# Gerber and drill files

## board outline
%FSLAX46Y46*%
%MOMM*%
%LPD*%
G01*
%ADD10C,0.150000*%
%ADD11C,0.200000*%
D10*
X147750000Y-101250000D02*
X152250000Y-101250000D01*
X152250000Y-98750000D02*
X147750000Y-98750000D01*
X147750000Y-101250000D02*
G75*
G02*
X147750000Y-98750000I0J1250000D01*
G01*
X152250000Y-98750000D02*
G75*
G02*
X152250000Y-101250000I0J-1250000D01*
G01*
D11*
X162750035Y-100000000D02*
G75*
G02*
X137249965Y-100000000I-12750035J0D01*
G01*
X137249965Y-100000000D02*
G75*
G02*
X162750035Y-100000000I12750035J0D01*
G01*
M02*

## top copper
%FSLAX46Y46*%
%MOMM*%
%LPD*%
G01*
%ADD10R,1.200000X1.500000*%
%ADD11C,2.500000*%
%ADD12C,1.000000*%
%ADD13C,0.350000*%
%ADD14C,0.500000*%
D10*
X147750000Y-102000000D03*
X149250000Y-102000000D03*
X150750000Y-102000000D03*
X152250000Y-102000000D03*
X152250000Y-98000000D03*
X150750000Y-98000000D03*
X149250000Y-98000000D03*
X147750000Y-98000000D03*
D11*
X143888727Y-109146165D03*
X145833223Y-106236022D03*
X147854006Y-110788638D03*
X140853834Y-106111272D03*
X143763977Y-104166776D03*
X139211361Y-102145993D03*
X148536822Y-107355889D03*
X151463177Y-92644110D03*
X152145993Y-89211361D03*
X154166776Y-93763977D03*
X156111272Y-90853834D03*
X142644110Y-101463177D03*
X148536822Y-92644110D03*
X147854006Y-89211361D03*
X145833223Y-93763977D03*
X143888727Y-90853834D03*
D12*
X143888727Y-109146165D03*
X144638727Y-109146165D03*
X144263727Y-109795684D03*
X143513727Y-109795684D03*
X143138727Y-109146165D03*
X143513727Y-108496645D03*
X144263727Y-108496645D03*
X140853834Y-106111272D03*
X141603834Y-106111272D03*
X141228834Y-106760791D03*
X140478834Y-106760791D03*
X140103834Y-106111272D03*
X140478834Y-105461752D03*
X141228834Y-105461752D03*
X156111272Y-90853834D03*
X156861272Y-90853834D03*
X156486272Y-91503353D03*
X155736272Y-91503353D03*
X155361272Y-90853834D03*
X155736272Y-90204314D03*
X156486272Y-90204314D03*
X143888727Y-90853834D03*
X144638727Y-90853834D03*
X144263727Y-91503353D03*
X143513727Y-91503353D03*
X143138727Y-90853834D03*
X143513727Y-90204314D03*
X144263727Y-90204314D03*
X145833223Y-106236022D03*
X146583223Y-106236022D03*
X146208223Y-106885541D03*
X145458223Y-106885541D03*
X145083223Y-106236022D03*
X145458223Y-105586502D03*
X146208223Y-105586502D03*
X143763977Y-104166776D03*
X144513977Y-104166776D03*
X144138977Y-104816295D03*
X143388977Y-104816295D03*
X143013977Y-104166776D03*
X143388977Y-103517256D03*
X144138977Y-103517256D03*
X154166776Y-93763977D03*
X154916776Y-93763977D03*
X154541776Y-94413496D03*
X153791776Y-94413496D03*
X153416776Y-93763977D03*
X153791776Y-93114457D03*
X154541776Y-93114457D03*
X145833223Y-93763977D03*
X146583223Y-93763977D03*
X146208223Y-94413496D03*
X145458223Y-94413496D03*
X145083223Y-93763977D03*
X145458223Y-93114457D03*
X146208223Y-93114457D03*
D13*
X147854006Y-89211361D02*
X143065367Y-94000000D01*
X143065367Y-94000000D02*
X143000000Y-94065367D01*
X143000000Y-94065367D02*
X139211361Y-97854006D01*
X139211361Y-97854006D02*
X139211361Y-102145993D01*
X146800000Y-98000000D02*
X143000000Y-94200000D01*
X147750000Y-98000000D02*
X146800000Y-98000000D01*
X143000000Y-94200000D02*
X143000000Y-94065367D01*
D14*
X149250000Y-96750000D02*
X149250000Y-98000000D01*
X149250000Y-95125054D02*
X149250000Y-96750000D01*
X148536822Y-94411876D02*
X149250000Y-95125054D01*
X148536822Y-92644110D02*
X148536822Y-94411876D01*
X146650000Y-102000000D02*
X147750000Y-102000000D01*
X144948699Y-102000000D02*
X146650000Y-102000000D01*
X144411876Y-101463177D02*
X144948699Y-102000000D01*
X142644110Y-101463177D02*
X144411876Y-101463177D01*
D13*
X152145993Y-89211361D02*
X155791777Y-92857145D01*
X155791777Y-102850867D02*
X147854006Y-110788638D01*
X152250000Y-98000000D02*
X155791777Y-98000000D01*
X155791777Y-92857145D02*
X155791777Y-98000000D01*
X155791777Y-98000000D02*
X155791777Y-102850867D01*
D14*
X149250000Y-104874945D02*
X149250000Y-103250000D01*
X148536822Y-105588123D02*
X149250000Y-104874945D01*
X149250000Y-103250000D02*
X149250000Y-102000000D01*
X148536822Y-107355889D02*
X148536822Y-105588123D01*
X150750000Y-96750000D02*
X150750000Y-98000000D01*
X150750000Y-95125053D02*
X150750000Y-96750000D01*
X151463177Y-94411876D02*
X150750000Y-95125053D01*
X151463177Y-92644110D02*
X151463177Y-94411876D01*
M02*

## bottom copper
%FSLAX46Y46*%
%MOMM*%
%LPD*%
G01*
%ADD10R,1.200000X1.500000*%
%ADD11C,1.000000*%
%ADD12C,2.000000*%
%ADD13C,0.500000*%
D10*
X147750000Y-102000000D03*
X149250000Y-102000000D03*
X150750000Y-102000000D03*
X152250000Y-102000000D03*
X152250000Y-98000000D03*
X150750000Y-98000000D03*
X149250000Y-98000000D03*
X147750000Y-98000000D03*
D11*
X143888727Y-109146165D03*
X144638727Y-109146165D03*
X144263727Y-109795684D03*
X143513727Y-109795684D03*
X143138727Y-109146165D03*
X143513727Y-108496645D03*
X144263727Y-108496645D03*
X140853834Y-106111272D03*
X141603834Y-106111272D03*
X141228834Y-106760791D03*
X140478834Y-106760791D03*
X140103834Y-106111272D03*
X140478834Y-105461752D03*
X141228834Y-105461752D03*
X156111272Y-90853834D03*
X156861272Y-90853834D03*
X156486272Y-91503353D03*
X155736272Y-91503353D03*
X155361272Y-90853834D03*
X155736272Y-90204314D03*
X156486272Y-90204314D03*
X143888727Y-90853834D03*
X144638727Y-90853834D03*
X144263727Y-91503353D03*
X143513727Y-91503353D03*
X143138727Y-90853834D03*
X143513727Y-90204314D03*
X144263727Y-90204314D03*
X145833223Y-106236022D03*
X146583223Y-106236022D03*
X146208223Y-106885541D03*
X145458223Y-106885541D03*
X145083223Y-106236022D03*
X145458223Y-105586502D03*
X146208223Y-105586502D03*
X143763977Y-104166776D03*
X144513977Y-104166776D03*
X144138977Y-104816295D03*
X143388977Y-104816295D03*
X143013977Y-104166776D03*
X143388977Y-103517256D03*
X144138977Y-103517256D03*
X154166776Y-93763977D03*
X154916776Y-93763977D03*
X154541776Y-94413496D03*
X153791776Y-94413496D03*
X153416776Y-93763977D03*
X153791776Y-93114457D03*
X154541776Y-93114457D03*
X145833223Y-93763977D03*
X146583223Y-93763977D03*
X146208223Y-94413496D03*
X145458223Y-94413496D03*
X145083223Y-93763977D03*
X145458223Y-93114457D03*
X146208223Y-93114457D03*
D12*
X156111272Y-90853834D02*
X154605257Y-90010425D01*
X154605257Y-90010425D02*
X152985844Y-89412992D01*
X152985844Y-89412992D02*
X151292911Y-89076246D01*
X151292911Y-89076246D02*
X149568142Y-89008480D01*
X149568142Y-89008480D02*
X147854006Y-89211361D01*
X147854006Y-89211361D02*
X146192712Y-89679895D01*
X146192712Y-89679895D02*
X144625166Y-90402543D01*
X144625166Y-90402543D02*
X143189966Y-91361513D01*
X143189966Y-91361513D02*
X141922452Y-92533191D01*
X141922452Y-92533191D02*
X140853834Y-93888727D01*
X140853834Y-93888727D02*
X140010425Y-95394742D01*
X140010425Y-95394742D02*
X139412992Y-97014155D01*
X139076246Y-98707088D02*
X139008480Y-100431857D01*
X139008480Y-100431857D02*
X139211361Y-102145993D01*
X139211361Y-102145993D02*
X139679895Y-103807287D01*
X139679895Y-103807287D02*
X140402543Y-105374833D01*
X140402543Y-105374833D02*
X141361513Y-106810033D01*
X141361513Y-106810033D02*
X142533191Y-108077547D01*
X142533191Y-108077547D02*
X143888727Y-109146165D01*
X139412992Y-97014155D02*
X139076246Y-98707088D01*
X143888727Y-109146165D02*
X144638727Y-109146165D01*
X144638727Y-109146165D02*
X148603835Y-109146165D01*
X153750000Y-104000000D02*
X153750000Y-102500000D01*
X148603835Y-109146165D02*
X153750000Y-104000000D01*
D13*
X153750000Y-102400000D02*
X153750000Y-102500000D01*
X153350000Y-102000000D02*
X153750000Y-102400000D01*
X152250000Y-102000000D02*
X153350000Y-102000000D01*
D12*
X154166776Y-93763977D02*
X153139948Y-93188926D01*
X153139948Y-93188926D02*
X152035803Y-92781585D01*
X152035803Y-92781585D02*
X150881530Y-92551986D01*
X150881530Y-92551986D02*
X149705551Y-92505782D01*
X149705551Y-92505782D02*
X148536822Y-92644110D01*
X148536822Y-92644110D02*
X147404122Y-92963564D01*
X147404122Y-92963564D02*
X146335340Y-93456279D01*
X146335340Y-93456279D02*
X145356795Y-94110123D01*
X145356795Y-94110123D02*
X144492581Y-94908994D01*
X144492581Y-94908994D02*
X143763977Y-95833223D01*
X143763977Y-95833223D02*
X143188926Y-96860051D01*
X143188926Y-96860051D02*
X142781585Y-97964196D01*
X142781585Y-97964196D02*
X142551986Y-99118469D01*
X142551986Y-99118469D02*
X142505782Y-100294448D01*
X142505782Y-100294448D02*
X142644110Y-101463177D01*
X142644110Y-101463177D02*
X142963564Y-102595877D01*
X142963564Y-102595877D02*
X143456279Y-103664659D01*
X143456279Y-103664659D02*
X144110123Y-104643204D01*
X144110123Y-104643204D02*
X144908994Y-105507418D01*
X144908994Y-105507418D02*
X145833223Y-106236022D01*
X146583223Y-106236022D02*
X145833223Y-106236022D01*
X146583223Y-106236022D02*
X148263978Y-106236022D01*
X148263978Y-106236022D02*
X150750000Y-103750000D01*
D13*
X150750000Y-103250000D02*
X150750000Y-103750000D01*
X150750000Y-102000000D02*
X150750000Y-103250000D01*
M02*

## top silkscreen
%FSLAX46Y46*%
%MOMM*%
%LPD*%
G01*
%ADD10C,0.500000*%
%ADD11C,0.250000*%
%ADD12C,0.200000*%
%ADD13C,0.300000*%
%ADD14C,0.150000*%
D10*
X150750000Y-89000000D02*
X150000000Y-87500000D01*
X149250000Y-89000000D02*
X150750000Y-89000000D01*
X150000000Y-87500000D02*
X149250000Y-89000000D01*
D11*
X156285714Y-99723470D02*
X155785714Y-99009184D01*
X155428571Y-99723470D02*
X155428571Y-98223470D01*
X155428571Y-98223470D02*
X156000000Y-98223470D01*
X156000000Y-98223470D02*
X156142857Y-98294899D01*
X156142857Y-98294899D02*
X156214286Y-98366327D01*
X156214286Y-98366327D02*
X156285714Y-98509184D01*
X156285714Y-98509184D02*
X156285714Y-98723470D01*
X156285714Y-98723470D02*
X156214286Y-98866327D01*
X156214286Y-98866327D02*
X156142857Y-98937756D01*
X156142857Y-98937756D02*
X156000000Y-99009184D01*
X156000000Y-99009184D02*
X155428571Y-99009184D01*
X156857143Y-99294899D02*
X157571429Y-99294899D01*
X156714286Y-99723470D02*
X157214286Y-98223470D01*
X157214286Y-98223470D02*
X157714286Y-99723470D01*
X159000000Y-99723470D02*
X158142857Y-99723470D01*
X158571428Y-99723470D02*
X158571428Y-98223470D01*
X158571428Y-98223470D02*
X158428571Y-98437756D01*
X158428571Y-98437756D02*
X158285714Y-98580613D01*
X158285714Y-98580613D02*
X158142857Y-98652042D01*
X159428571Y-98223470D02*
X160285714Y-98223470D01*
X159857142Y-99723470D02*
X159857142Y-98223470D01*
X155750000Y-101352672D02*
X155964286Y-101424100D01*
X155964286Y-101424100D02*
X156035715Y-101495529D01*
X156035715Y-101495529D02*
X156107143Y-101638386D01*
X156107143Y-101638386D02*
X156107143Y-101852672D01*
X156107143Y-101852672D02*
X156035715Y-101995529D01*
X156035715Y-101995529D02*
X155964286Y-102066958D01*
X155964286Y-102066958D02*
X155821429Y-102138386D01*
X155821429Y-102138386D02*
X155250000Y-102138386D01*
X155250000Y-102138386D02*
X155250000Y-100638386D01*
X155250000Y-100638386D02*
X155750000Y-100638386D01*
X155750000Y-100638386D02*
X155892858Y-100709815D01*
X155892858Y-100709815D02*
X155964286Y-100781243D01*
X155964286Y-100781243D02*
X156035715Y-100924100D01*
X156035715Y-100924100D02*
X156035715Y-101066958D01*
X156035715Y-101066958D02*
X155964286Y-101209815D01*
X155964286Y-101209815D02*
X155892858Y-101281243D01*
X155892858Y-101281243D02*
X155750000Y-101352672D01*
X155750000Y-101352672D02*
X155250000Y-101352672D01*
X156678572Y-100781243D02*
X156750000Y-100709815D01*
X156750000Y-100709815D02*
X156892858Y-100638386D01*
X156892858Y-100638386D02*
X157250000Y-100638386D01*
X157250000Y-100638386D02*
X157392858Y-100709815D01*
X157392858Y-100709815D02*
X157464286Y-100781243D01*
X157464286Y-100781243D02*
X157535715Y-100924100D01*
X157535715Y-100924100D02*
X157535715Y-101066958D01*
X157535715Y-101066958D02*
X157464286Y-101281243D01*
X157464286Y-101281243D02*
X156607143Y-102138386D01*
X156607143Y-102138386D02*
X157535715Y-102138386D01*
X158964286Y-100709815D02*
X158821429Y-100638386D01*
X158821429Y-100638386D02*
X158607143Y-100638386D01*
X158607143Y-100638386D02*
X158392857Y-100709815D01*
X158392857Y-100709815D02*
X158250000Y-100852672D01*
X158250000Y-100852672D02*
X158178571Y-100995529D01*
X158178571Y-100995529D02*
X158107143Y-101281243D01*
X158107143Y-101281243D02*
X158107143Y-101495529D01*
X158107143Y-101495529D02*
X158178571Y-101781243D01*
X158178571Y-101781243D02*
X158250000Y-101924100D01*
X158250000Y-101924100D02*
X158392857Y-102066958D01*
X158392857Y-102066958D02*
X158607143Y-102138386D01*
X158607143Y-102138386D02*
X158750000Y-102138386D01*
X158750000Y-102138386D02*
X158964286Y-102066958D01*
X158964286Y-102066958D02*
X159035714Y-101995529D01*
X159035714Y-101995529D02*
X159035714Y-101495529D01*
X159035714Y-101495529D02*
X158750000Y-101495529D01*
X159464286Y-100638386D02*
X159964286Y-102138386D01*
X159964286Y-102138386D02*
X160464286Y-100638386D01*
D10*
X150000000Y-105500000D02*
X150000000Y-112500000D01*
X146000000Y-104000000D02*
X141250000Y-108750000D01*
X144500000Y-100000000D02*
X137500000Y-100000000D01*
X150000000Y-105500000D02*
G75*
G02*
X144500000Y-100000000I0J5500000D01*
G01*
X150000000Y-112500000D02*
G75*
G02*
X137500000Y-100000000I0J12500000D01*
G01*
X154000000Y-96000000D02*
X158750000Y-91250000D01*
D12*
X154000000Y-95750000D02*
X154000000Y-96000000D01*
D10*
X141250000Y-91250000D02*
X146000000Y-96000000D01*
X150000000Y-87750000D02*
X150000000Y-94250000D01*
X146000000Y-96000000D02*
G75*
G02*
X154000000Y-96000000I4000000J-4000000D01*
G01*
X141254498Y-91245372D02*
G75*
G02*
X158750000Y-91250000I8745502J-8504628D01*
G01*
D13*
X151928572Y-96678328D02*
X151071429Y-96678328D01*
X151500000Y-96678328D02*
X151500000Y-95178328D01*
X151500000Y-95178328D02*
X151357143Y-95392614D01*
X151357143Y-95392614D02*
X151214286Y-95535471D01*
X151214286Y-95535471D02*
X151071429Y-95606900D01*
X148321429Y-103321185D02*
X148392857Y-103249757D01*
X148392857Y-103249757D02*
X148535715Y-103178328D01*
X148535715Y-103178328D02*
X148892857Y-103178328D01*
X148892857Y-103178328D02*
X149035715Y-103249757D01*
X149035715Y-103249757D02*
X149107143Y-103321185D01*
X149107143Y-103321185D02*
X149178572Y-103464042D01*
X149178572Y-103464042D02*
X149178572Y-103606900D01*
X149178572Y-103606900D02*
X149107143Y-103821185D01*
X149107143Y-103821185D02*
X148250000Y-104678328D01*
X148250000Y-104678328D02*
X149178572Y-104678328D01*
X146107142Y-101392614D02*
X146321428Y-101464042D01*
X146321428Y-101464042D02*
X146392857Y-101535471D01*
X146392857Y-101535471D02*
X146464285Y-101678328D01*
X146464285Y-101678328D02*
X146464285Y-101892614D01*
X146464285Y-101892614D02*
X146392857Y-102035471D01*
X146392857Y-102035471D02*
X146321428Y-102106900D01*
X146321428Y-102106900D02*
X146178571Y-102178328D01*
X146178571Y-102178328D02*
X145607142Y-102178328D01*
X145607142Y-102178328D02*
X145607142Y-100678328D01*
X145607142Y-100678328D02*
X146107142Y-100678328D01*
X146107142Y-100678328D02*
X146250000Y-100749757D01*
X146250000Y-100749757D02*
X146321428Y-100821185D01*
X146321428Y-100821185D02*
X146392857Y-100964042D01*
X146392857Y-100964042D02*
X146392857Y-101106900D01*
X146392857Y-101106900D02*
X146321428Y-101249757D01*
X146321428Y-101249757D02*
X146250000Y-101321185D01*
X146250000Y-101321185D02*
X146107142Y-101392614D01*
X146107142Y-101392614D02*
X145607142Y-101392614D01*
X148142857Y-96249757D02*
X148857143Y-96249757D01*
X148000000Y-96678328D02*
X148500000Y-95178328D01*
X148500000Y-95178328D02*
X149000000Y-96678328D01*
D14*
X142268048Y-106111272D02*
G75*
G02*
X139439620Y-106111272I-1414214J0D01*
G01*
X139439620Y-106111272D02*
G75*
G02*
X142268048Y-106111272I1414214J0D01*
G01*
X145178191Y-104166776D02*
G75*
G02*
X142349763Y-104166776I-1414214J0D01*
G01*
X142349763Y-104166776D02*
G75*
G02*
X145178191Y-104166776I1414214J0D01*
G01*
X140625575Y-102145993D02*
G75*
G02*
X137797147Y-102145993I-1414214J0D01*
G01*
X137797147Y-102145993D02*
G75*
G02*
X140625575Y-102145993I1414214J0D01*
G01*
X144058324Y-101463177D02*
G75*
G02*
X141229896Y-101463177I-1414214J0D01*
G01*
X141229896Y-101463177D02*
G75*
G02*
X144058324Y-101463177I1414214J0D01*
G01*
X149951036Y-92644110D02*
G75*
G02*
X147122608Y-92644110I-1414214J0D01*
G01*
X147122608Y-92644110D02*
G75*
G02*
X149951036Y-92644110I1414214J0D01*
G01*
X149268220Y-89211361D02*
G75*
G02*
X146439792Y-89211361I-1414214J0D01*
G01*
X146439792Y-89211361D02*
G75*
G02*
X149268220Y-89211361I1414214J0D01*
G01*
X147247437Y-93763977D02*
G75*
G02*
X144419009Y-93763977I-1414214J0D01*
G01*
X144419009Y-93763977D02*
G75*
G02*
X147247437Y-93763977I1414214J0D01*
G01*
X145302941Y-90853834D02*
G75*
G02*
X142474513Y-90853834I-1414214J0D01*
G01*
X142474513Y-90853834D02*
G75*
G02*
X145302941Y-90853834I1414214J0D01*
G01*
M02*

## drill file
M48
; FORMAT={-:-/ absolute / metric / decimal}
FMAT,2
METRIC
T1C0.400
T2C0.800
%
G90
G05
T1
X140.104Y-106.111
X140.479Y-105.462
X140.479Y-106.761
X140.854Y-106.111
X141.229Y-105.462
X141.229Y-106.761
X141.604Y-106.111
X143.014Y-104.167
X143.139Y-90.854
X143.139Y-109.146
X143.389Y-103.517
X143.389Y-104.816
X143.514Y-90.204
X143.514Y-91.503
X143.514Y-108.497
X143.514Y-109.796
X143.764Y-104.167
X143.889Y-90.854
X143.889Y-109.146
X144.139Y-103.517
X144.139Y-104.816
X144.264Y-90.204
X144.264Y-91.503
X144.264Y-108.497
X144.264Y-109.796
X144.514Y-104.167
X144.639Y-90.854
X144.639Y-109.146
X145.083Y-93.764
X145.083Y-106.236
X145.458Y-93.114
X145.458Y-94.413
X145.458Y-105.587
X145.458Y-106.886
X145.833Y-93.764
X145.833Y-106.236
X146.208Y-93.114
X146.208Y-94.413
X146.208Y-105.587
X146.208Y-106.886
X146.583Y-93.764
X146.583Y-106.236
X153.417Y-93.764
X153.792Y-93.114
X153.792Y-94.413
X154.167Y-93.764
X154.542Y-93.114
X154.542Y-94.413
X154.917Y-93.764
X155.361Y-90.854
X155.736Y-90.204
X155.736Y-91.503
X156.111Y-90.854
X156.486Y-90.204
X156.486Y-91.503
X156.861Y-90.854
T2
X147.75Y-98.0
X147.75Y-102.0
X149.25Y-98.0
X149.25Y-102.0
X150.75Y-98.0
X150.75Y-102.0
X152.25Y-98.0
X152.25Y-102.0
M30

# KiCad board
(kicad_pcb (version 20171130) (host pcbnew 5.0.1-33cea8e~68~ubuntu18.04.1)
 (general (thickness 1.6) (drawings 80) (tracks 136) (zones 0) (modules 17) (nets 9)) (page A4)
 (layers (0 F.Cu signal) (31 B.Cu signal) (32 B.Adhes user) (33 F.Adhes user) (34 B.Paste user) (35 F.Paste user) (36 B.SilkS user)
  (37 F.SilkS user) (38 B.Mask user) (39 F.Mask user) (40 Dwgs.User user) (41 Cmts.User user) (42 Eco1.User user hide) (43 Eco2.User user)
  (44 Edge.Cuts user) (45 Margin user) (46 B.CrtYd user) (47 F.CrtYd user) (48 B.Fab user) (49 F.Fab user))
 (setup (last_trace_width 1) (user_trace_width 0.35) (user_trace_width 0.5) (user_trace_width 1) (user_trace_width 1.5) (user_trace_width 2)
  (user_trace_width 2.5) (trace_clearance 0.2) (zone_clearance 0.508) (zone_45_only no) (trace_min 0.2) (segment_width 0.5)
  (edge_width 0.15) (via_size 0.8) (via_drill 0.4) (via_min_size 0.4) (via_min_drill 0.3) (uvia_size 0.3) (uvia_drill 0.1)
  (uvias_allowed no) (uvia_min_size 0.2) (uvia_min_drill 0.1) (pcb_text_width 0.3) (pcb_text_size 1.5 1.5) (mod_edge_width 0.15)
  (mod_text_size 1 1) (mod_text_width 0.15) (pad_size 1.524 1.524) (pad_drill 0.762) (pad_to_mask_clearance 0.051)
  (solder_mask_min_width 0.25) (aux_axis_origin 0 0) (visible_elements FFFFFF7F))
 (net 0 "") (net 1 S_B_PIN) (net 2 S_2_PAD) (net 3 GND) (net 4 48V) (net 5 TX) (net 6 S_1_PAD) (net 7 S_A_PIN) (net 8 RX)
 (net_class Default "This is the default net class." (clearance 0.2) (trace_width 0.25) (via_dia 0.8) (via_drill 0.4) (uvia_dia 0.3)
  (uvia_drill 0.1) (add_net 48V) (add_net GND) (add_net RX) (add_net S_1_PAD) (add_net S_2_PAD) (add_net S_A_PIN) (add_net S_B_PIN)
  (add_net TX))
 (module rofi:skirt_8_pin (layer F.Cu) (at 150 100)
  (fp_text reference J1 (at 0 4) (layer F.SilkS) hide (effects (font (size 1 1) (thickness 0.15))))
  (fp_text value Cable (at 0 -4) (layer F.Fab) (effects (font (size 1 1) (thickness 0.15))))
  (pad 8 thru_hole rect (at -2.25 2) (size 1.2 1.5) (drill 0.8) (layers *.Cu *.Mask) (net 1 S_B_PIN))
  (pad 7 thru_hole rect (at -0.75 2) (size 1.2 1.5) (drill 0.8) (layers *.Cu *.Mask) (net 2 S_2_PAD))
  (pad 6 thru_hole rect (at 0.75 2) (size 1.2 1.5) (drill 0.8) (layers *.Cu *.Mask) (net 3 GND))
  (pad 5 thru_hole rect (at 2.25 2) (size 1.2 1.5) (drill 0.8) (layers *.Cu *.Mask) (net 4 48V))
  (pad 4 thru_hole rect (at 2.25 -2) (size 1.2 1.5) (drill 0.8) (layers *.Cu *.Mask) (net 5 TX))
  (pad 3 thru_hole rect (at 0.75 -2) (size 1.2 1.5) (drill 0.8) (layers *.Cu *.Mask) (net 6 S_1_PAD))
  (pad 2 thru_hole rect (at -0.75 -2) (size 1.2 1.5) (drill 0.8) (layers *.Cu *.Mask) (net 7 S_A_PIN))
  (pad 1 thru_hole rect (at -2.25 -2) (size 1.2 1.5) (drill 0.8) (layers *.Cu *.Mask) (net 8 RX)))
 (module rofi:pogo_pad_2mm (layer F.Cu) (at 143.888727 109.146165)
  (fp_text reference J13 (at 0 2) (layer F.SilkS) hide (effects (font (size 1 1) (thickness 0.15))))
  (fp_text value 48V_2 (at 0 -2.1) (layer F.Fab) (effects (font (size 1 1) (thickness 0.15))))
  (pad 1 smd circle (at 0 0) (size 2.5 2.5) (layers F.Cu F.Paste F.Mask) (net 4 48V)))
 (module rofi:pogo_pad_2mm (layer F.Cu) (at 145.833223 106.236022)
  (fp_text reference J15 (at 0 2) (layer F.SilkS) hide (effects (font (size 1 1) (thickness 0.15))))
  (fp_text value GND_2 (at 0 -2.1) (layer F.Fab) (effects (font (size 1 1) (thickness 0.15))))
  (pad 1 smd circle (at 0 0) (size 2.5 2.5) (layers F.Cu F.Paste F.Mask) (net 3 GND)))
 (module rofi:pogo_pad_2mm (layer F.Cu) (at 147.854006 110.788638)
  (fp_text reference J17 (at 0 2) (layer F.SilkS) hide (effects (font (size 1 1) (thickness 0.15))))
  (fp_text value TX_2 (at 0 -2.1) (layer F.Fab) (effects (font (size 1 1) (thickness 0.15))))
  (pad 1 smd circle (at 0 0) (size 2.5 2.5) (layers F.Cu F.Paste F.Mask) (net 5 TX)))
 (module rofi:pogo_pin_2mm (layer F.Cu) (at 140.853834 106.111272)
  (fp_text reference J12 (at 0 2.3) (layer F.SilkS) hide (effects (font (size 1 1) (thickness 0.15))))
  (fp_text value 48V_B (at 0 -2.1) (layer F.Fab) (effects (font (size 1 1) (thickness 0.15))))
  (fp_circle (center 0 0) (end 0.2 -1.4) (layer F.SilkS) (width 0.15))
  (pad 1 smd circle (at 0 0) (size 2.5 2.5) (layers F.Cu F.Paste F.Mask) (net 4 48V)))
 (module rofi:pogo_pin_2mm (layer F.Cu) (at 143.763977 104.166776)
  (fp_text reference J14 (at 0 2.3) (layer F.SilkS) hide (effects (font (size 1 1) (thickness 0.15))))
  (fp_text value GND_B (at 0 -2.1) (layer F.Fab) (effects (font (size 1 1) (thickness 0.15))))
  (fp_circle (center 0 0) (end 0.2 -1.4) (layer F.SilkS) (width 0.15))
  (pad 1 smd circle (at 0 0) (size 2.5 2.5) (layers F.Cu F.Paste F.Mask) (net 3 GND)))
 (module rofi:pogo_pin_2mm (layer F.Cu) (at 139.211361 102.145993)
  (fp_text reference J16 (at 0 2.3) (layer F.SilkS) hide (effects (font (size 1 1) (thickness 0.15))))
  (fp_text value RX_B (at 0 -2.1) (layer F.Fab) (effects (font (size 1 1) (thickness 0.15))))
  (fp_circle (center 0 0) (end 0.2 -1.4) (layer F.SilkS) (width 0.15))
  (pad 1 smd circle (at 0 0) (size 2.5 2.5) (layers F.Cu F.Paste F.Mask) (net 8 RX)))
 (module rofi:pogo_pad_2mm (layer F.Cu) (at 148.536822 107.355889)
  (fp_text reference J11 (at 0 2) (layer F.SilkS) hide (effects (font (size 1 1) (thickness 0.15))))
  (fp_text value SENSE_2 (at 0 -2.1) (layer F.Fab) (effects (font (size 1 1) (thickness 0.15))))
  (pad 1 smd circle (at 0 0) (size 2.5 2.5) (layers F.Cu F.Paste F.Mask) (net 2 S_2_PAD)))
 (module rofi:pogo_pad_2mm (layer F.Cu) (at 151.463177 92.64411)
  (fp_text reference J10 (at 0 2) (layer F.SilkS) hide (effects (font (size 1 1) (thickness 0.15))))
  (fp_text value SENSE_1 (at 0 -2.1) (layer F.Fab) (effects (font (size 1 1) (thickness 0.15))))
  (pad 1 smd circle (at 0 0) (size 2.5 2.5) (layers F.Cu F.Paste F.Mask) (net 6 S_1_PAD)))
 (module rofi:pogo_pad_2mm (layer F.Cu) (at 152.145993 89.211361)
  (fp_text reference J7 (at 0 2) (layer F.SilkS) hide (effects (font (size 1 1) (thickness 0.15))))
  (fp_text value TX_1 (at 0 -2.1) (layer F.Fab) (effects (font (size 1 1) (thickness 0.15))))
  (pad 1 smd circle (at 0 0) (size 2.5 2.5) (layers F.Cu F.Paste F.Mask) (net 5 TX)))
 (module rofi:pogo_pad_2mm (layer F.Cu) (at 154.166776 93.763977)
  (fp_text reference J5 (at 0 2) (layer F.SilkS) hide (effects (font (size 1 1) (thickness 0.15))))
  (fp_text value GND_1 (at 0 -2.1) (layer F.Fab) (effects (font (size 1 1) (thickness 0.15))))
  (pad 1 smd circle (at 0 0) (size 2.5 2.5) (layers F.Cu F.Paste F.Mask) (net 3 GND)))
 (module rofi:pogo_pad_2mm (layer F.Cu) (at 156.111272 90.853834)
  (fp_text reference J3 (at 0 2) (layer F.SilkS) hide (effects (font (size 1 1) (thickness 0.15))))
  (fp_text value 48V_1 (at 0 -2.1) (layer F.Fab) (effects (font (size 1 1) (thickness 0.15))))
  (pad 1 smd circle (at 0 0) (size 2.5 2.5) (layers F.Cu F.Paste F.Mask) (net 4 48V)))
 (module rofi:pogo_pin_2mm (layer F.Cu) (at 142.64411 101.463177)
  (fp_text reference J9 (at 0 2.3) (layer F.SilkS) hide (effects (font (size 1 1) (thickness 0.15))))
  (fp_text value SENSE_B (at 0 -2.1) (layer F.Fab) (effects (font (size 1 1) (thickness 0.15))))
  (fp_circle (center 0 0) (end 0.2 -1.4) (layer F.SilkS) (width 0.15))
  (pad 1 smd circle (at 0 0) (size 2.5 2.5) (layers F.Cu F.Paste F.Mask) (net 1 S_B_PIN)))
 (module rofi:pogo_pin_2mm (layer F.Cu) (at 148.536822 92.64411)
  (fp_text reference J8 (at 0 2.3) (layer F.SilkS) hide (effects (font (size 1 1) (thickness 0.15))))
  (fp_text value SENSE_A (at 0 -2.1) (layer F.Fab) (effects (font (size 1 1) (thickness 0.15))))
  (fp_circle (center 0 0) (end 0.2 -1.4) (layer F.SilkS) (width 0.15))
  (pad 1 smd circle (at 0 0) (size 2.5 2.5) (layers F.Cu F.Paste F.Mask) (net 7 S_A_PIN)))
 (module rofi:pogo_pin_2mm (layer F.Cu) (at 147.854006 89.211361)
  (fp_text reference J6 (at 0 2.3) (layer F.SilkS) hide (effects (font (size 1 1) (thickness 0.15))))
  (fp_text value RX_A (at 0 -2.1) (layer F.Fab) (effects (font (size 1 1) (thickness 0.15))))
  (fp_circle (center 0 0) (end 0.2 -1.4) (layer F.SilkS) (width 0.15))
  (pad 1 smd circle (at 0 0) (size 2.5 2.5) (layers F.Cu F.Paste F.Mask) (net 8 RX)))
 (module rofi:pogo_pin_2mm (layer F.Cu) (at 145.833223 93.763977)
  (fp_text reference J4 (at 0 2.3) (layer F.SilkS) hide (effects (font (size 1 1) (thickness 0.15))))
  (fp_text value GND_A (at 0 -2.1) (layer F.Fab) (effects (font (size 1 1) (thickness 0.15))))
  (fp_circle (center 0 0) (end 0.2 -1.4) (layer F.SilkS) (width 0.15))
  (pad 1 smd circle (at 0 0) (size 2.5 2.5) (layers F.Cu F.Paste F.Mask) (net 3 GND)))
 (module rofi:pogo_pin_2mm (layer F.Cu) (at 143.888727 90.853834)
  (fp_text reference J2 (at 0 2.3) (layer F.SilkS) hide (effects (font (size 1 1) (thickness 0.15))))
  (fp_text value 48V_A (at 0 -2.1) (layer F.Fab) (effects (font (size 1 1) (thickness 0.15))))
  (fp_circle (center 0 0) (end 0.2 -1.4) (layer F.SilkS) (width 0.15))
  (pad 1 smd circle (at 0 0) (size 2.5 2.5) (layers F.Cu F.Paste F.Mask) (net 4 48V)))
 (gr_line (start 150.75 89) (end 150 87.5) (layer F.SilkS) (width 0.5))
 (gr_line (start 149.25 89) (end 150.75 89) (layer F.SilkS) (width 0.5))
 (gr_line (start 150 87.5) (end 149.25 89) (layer F.SilkS) (width 0.5))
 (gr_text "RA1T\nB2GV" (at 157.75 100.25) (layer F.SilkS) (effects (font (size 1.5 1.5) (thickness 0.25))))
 (gr_line (start 150 105.5) (end 150 112.5) (layer F.SilkS) (width 0.5))
 (gr_line (start 146 104) (end 141.25 108.75) (layer F.SilkS) (width 0.5))
 (gr_line (start 144.5 100) (end 137.5 100) (layer F.SilkS) (width 0.5))
 (gr_arc (start 150 100) (end 144.5 100) (angle -90) (layer F.SilkS) (width 0.5))
 (gr_arc (start 150 100) (end 137.5 100) (angle -90) (layer F.SilkS) (width 0.5))
 (gr_line (start 154 96) (end 158.75 91.25) (layer F.SilkS) (width 0.5))
 (gr_line (start 154 95.75) (end 154 96) (layer F.SilkS) (width 0.2))
 (gr_line (start 141.25 91.25) (end 146 96) (layer F.SilkS) (width 0.5))
 (gr_line (start 150 87.75) (end 150 94.25) (layer F.SilkS) (width 0.5))
 (gr_arc (start 150 100) (end 154 96) (angle -90) (layer F.SilkS) (width 0.5))
 (gr_arc (start 150 99.75) (end 158.75 91.25) (angle -91.63031912) (layer F.SilkS) (width 0.5))
 (gr_line (start 147.75 101.25) (end 152.25 101.25) (layer Edge.Cuts) (width 0.15))
 (gr_line (start 152.25 98.75) (end 147.75 98.75) (layer Edge.Cuts) (width 0.15))
 (gr_arc (start 147.75 100) (end 147.75 98.75) (angle -180) (layer Edge.Cuts) (width 0.15))
 (gr_arc (start 152.25 100) (end 152.25 101.25) (angle -180) (layer Edge.Cuts) (width 0.15))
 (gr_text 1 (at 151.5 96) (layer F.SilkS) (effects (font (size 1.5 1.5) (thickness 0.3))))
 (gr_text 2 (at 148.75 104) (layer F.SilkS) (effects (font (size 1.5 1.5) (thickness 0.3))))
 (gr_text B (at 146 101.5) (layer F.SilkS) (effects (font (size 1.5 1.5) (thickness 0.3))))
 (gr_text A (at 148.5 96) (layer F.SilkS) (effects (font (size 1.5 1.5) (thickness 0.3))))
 (gr_circle (center 150 100) (end 162.750035 100) (layer Edge.Cuts) (width 0.2))
 (via (at 143.888727 109.146165) (size 1) (layers F.Cu B.Cu) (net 4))
 (via (at 144.638727 109.146165) (size 1) (layers F.Cu B.Cu) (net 4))
 (via (at 144.263727 109.795684) (size 1) (layers F.Cu B.Cu) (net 4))
 (via (at 143.513727 109.795684) (size 1) (layers F.Cu B.Cu) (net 4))
 (via (at 143.138727 109.146165) (size 1) (layers F.Cu B.Cu) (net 4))
 (via (at 143.513727 108.496645) (size 1) (layers F.Cu B.Cu) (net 4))
 (via (at 144.263727 108.496645) (size 1) (layers F.Cu B.Cu) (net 4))
 (via (at 140.853834 106.111272) (size 1) (layers F.Cu B.Cu) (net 4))
 (via (at 141.603834 106.111272) (size 1) (layers F.Cu B.Cu) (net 4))
 (via (at 141.228834 106.760791) (size 1) (layers F.Cu B.Cu) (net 4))
 (via (at 140.478834 106.760791) (size 1) (layers F.Cu B.Cu) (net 4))
 (via (at 140.103834 106.111272) (size 1) (layers F.Cu B.Cu) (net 4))
 (via (at 140.478834 105.461752) (size 1) (layers F.Cu B.Cu) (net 4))
 (via (at 141.228834 105.461752) (size 1) (layers F.Cu B.Cu) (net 4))
 (via (at 156.111272 90.853834) (size 1) (layers F.Cu B.Cu) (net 4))
 (via (at 156.861272 90.853834) (size 1) (layers F.Cu B.Cu) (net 4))
 (via (at 156.486272 91.503353) (size 1) (layers F.Cu B.Cu) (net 4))
 (via (at 155.736272 91.503353) (size 1) (layers F.Cu B.Cu) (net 4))
 (via (at 155.361272 90.853834) (size 1) (layers F.Cu B.Cu) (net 4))
 (via (at 155.736272 90.204314) (size 1) (layers F.Cu B.Cu) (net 4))
 (via (at 156.486272 90.204314) (size 1) (layers F.Cu B.Cu) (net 4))
 (via (at 143.888727 90.853834) (size 1) (layers F.Cu B.Cu) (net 4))
 (via (at 144.638727 90.853834) (size 1) (layers F.Cu B.Cu) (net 4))
 (via (at 144.263727 91.503353) (size 1) (layers F.Cu B.Cu) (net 4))
 (via (at 143.513727 91.503353) (size 1) (layers F.Cu B.Cu) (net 4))
 (via (at 143.138727 90.853834) (size 1) (layers F.Cu B.Cu) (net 4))
 (via (at 143.513727 90.204314) (size 1) (layers F.Cu B.Cu) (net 4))
 (via (at 144.263727 90.204314) (size 1) (layers F.Cu B.Cu) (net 4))
 (segment (start 156.111272 90.853834) (end 154.605257 90.010425) (width 2) (layer B.Cu) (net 4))
 (segment (start 154.605257 90.010425) (end 152.985844 89.412992) (width 2) (layer B.Cu) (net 4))
 (segment (start 152.985844 89.412992) (end 151.292911 89.076246) (width 2) (layer B.Cu) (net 4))
 (segment (start 151.292911 89.076246) (end 149.568142 89.00848) (width 2) (layer B.Cu) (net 4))
 (segment (start 149.568142 89.00848) (end 147.854006 89.211361) (width 2) (layer B.Cu) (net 4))
 (segment (start 147.854006 89.211361) (end 146.192712 89.679895) (width 2) (layer B.Cu) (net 4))
 (segment (start 146.192712 89.679895) (end 144.625166 90.402543) (width 2) (layer B.Cu) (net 4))
 (segment (start 144.625166 90.402543) (end 143.189966 91.361513) (width 2) (layer B.Cu) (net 4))
 (segment (start 143.189966 91.361513) (end 141.922452 92.533191) (width 2) (layer B.Cu) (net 4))
 (segment (start 141.922452 92.533191) (end 140.853834 93.888727) (width 2) (layer B.Cu) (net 4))
 (segment (start 140.853834 93.888727) (end 140.010425 95.394742) (width 2) (layer B.Cu) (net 4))
 (segment (start 140.010425 95.394742) (end 139.412992 97.014155) (width 2) (layer B.Cu) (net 4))
 (segment (start 139.076246 98.707088) (end 139.00848 100.431857) (width 2) (layer B.Cu) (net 4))
 (segment (start 139.00848 100.431857) (end 139.211361 102.145993) (width 2) (layer B.Cu) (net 4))
 (segment (start 139.211361 102.145993) (end 139.679895 103.807287) (width 2) (layer B.Cu) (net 4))
 (segment (start 139.679895 103.807287) (end 140.402543 105.374833) (width 2) (layer B.Cu) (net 4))
 (segment (start 140.402543 105.374833) (end 141.361513 106.810033) (width 2) (layer B.Cu) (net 4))
 (segment (start 141.361513 106.810033) (end 142.533191 108.077547) (width 2) (layer B.Cu) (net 4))
 (segment (start 142.533191 108.077547) (end 143.888727 109.146165) (width 2) (layer B.Cu) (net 4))
 (segment (start 139.412992 97.014155) (end 139.076246 98.707088) (width 2) (layer B.Cu) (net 4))
 (segment (start 143.888727 109.146165) (end 144.638727 109.146165) (width 2) (layer B.Cu) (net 4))
 (segment (start 144.638727 109.146165) (end 148.603835 109.146165) (width 2) (layer B.Cu) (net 4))
 (segment (start 153.75 104) (end 153.75 102.5) (width 2) (layer B.Cu) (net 4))
 (segment (start 148.603835 109.146165) (end 153.75 104) (width 2) (layer B.Cu) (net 4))
 (segment (start 153.75 102.4) (end 153.75 102.5) (width 0.5) (layer B.Cu) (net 4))
 (segment (start 153.35 102) (end 153.75 102.4) (width 0.5) (layer B.Cu) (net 4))
 (segment (start 152.25 102) (end 153.35 102) (width 0.5) (layer B.Cu) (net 4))
 (via (at 145.833223 106.236022) (size 1) (layers F.Cu B.Cu) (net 3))
 (via (at 146.583223 106.236022) (size 1) (layers F.Cu B.Cu) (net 3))
 (via (at 146.208223 106.885541) (size 1) (layers F.Cu B.Cu) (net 3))
 (via (at 145.458223 106.885541) (size 1) (layers F.Cu B.Cu) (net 3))
 (via (at 145.083223 106.236022) (size 1) (layers F.Cu B.Cu) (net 3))
 (via (at 145.458223 105.586502) (size 1) (layers F.Cu B.Cu) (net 3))
 (via (at 146.208223 105.586502) (size 1) (layers F.Cu B.Cu) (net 3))
 (via (at 143.763977 104.166776) (size 1) (layers F.Cu B.Cu) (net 3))
 (via (at 144.513977 104.166776) (size 1) (layers F.Cu B.Cu) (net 3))
 (via (at 144.138977 104.816295) (size 1) (layers F.Cu B.Cu) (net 3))
 (via (at 143.388977 104.816295) (size 1) (layers F.Cu B.Cu) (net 3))
 (via (at 143.013977 104.166776) (size 1) (layers F.Cu B.Cu) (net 3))
 (via (at 143.388977 103.517256) (size 1) (layers F.Cu B.Cu) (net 3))
 (via (at 144.138977 103.517256) (size 1) (layers F.Cu B.Cu) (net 3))
 (via (at 154.166776 93.763977) (size 1) (layers F.Cu B.Cu) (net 3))
 (via (at 154.916776 93.763977) (size 1) (layers F.Cu B.Cu) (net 3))
 (via (at 154.541776 94.413496) (size 1) (layers F.Cu B.Cu) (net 3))
 (via (at 153.791776 94.413496) (size 1) (layers F.Cu B.Cu) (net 3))
 (via (at 153.416776 93.763977) (size 1) (layers F.Cu B.Cu) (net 3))
 (via (at 153.791776 93.114457) (size 1) (layers F.Cu B.Cu) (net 3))
 (via (at 154.541776 93.114457) (size 1) (layers F.Cu B.Cu) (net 3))
 (via (at 145.833223 93.763977) (size 1) (layers F.Cu B.Cu) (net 3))
 (via (at 146.583223 93.763977) (size 1) (layers F.Cu B.Cu) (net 3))
 (via (at 146.208223 94.413496) (size 1) (layers F.Cu B.Cu) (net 3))
 (via (at 145.458223 94.413496) (size 1) (layers F.Cu B.Cu) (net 3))
 (via (at 145.083223 93.763977) (size 1) (layers F.Cu B.Cu) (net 3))
 (via (at 145.458223 93.114457) (size 1) (layers F.Cu B.Cu) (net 3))
 (via (at 146.208223 93.114457) (size 1) (layers F.Cu B.Cu) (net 3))
 (segment (start 154.166776 93.763977) (end 153.139948 93.188926) (width 2) (layer B.Cu) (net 3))
 (segment (start 153.139948 93.188926) (end 152.035803 92.781585) (width 2) (layer B.Cu) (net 3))
 (segment (start 152.035803 92.781585) (end 150.88153 92.551986) (width 2) (layer B.Cu) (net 3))
 (segment (start 150.88153 92.551986) (end 149.705551 92.505782) (width 2) (layer B.Cu) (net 3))
 (segment (start 149.705551 92.505782) (end 148.536822 92.64411) (width 2) (layer B.Cu) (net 3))
 (segment (start 148.536822 92.64411) (end 147.404122 92.963564) (width 2) (layer B.Cu) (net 3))
 (segment (start 147.404122 92.963564) (end 146.33534 93.456279) (width 2) (layer B.Cu) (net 3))
 (segment (start 146.33534 93.456279) (end 145.356795 94.110123) (width 2) (layer B.Cu) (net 3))
 (segment (start 145.356795 94.110123) (end 144.492581 94.908994) (width 2) (layer B.Cu) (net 3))
 (segment (start 144.492581 94.908994) (end 143.763977 95.833223) (width 2) (layer B.Cu) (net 3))
 (segment (start 143.763977 95.833223) (end 143.188926 96.860051) (width 2) (layer B.Cu) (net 3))
 (segment (start 143.188926 96.860051) (end 142.781585 97.964196) (width 2) (layer B.Cu) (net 3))
 (segment (start 142.781585 97.964196) (end 142.551986 99.118469) (width 2) (layer B.Cu) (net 3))
 (segment (start 142.551986 99.118469) (end 142.505782 100.294448) (width 2) (layer B.Cu) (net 3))
 (segment (start 142.505782 100.294448) (end 142.64411 101.463177) (width 2) (layer B.Cu) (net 3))
 (segment (start 142.64411 101.463177) (end 142.963564 102.595877) (width 2) (layer B.Cu) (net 3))
 (segment (start 142.963564 102.595877) (end 143.456279 103.664659) (width 2) (layer B.Cu) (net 3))
 (segment (start 143.456279 103.664659) (end 144.110123 104.643204) (width 2) (layer B.Cu) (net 3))
 (segment (start 144.110123 104.643204) (end 144.908994 105.507418) (width 2) (layer B.Cu) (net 3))
 (segment (start 144.908994 105.507418) (end 145.833223 106.236022) (width 2) (layer B.Cu) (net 3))
 (segment (start 146.583223 106.236022) (end 145.833223 106.236022) (width 2) (layer B.Cu) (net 3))
 (segment (start 146.583223 106.236022) (end 148.263978 106.236022) (width 2) (layer B.Cu) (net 3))
 (segment (start 148.263978 106.236022) (end 150.75 103.75) (width 2) (layer B.Cu) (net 3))
 (segment (start 150.75 103.25) (end 150.75 103.75) (width 0.5) (layer B.Cu) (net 3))
 (segment (start 150.75 102) (end 150.75 103.25) (width 0.5) (layer B.Cu) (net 3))
 (segment (start 147.854006 89.211361) (end 143.065367 94) (width 0.35) (layer F.Cu) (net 8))
 (segment (start 143.065367 94) (end 143 94.065367) (width 0.35) (layer F.Cu) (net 8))
 (segment (start 143 94.065367) (end 139.211361 97.854006) (width 0.35) (layer F.Cu) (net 8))
 (segment (start 139.211361 97.854006) (end 139.211361 102.145993) (width 0.35) (layer F.Cu) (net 8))
 (segment (start 146.8 98) (end 143 94.2) (width 0.35) (layer F.Cu) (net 8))
 (segment (start 147.75 98) (end 146.8 98) (width 0.35) (layer F.Cu) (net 8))
 (segment (start 143 94.2) (end 143 94.065367) (width 0.35) (layer F.Cu) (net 8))
 (segment (start 149.25 96.75) (end 149.25 98) (width 0.5) (layer F.Cu) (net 7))
 (segment (start 149.25 95.125054) (end 149.25 96.75) (width 0.5) (layer F.Cu) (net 7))
 (segment (start 148.536822 94.411876) (end 149.25 95.125054) (width 0.5) (layer F.Cu) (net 7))
 (segment (start 148.536822 92.64411) (end 148.536822 94.411876) (width 0.5) (layer F.Cu) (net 7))
 (segment (start 146.65 102) (end 147.75 102) (width 0.5) (layer F.Cu) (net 1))
 (segment (start 144.948699 102) (end 146.65 102) (width 0.5) (layer F.Cu) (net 1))
 (segment (start 144.411876 101.463177) (end 144.948699 102) (width 0.5) (layer F.Cu) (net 1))
 (segment (start 142.64411 101.463177) (end 144.411876 101.463177) (width 0.5) (layer F.Cu) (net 1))
 (segment (start 152.145993 89.211361) (end 155.791777 92.857145) (width 0.35) (layer F.Cu) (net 5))
 (segment (start 155.791777 102.850867) (end 147.854006 110.788638) (width 0.35) (layer F.Cu) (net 5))
 (segment (start 152.25 98) (end 155.791777 98) (width 0.35) (layer F.Cu) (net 5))
 (segment (start 155.791777 92.857145) (end 155.791777 98) (width 0.35) (layer F.Cu) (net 5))
 (segment (start 155.791777 98) (end 155.791777 102.850867) (width 0.35) (layer F.Cu) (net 5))
 (segment (start 149.25 104.874945) (end 149.25 103.25) (width 0.5) (layer F.Cu) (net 2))
 (segment (start 148.536822 105.588123) (end 149.25 104.874945) (width 0.5) (layer F.Cu) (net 2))
 (segment (start 149.25 103.25) (end 149.25 102) (width 0.5) (layer F.Cu) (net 2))
 (segment (start 148.536822 107.355889) (end 148.536822 105.588123) (width 0.5) (layer F.Cu) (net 2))
 (segment (start 150.75 96.75) (end 150.75 98) (width 0.5) (layer F.Cu) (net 6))
 (segment (start 150.75 95.125053) (end 150.75 96.75) (width 0.5) (layer F.Cu) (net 6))
 (segment (start 151.463177 94.411876) (end 150.75 95.125053) (width 0.5) (layer F.Cu) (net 6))
 (segment (start 151.463177 92.64411) (end 151.463177 94.411876) (width 0.5) (layer F.Cu) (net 6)))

